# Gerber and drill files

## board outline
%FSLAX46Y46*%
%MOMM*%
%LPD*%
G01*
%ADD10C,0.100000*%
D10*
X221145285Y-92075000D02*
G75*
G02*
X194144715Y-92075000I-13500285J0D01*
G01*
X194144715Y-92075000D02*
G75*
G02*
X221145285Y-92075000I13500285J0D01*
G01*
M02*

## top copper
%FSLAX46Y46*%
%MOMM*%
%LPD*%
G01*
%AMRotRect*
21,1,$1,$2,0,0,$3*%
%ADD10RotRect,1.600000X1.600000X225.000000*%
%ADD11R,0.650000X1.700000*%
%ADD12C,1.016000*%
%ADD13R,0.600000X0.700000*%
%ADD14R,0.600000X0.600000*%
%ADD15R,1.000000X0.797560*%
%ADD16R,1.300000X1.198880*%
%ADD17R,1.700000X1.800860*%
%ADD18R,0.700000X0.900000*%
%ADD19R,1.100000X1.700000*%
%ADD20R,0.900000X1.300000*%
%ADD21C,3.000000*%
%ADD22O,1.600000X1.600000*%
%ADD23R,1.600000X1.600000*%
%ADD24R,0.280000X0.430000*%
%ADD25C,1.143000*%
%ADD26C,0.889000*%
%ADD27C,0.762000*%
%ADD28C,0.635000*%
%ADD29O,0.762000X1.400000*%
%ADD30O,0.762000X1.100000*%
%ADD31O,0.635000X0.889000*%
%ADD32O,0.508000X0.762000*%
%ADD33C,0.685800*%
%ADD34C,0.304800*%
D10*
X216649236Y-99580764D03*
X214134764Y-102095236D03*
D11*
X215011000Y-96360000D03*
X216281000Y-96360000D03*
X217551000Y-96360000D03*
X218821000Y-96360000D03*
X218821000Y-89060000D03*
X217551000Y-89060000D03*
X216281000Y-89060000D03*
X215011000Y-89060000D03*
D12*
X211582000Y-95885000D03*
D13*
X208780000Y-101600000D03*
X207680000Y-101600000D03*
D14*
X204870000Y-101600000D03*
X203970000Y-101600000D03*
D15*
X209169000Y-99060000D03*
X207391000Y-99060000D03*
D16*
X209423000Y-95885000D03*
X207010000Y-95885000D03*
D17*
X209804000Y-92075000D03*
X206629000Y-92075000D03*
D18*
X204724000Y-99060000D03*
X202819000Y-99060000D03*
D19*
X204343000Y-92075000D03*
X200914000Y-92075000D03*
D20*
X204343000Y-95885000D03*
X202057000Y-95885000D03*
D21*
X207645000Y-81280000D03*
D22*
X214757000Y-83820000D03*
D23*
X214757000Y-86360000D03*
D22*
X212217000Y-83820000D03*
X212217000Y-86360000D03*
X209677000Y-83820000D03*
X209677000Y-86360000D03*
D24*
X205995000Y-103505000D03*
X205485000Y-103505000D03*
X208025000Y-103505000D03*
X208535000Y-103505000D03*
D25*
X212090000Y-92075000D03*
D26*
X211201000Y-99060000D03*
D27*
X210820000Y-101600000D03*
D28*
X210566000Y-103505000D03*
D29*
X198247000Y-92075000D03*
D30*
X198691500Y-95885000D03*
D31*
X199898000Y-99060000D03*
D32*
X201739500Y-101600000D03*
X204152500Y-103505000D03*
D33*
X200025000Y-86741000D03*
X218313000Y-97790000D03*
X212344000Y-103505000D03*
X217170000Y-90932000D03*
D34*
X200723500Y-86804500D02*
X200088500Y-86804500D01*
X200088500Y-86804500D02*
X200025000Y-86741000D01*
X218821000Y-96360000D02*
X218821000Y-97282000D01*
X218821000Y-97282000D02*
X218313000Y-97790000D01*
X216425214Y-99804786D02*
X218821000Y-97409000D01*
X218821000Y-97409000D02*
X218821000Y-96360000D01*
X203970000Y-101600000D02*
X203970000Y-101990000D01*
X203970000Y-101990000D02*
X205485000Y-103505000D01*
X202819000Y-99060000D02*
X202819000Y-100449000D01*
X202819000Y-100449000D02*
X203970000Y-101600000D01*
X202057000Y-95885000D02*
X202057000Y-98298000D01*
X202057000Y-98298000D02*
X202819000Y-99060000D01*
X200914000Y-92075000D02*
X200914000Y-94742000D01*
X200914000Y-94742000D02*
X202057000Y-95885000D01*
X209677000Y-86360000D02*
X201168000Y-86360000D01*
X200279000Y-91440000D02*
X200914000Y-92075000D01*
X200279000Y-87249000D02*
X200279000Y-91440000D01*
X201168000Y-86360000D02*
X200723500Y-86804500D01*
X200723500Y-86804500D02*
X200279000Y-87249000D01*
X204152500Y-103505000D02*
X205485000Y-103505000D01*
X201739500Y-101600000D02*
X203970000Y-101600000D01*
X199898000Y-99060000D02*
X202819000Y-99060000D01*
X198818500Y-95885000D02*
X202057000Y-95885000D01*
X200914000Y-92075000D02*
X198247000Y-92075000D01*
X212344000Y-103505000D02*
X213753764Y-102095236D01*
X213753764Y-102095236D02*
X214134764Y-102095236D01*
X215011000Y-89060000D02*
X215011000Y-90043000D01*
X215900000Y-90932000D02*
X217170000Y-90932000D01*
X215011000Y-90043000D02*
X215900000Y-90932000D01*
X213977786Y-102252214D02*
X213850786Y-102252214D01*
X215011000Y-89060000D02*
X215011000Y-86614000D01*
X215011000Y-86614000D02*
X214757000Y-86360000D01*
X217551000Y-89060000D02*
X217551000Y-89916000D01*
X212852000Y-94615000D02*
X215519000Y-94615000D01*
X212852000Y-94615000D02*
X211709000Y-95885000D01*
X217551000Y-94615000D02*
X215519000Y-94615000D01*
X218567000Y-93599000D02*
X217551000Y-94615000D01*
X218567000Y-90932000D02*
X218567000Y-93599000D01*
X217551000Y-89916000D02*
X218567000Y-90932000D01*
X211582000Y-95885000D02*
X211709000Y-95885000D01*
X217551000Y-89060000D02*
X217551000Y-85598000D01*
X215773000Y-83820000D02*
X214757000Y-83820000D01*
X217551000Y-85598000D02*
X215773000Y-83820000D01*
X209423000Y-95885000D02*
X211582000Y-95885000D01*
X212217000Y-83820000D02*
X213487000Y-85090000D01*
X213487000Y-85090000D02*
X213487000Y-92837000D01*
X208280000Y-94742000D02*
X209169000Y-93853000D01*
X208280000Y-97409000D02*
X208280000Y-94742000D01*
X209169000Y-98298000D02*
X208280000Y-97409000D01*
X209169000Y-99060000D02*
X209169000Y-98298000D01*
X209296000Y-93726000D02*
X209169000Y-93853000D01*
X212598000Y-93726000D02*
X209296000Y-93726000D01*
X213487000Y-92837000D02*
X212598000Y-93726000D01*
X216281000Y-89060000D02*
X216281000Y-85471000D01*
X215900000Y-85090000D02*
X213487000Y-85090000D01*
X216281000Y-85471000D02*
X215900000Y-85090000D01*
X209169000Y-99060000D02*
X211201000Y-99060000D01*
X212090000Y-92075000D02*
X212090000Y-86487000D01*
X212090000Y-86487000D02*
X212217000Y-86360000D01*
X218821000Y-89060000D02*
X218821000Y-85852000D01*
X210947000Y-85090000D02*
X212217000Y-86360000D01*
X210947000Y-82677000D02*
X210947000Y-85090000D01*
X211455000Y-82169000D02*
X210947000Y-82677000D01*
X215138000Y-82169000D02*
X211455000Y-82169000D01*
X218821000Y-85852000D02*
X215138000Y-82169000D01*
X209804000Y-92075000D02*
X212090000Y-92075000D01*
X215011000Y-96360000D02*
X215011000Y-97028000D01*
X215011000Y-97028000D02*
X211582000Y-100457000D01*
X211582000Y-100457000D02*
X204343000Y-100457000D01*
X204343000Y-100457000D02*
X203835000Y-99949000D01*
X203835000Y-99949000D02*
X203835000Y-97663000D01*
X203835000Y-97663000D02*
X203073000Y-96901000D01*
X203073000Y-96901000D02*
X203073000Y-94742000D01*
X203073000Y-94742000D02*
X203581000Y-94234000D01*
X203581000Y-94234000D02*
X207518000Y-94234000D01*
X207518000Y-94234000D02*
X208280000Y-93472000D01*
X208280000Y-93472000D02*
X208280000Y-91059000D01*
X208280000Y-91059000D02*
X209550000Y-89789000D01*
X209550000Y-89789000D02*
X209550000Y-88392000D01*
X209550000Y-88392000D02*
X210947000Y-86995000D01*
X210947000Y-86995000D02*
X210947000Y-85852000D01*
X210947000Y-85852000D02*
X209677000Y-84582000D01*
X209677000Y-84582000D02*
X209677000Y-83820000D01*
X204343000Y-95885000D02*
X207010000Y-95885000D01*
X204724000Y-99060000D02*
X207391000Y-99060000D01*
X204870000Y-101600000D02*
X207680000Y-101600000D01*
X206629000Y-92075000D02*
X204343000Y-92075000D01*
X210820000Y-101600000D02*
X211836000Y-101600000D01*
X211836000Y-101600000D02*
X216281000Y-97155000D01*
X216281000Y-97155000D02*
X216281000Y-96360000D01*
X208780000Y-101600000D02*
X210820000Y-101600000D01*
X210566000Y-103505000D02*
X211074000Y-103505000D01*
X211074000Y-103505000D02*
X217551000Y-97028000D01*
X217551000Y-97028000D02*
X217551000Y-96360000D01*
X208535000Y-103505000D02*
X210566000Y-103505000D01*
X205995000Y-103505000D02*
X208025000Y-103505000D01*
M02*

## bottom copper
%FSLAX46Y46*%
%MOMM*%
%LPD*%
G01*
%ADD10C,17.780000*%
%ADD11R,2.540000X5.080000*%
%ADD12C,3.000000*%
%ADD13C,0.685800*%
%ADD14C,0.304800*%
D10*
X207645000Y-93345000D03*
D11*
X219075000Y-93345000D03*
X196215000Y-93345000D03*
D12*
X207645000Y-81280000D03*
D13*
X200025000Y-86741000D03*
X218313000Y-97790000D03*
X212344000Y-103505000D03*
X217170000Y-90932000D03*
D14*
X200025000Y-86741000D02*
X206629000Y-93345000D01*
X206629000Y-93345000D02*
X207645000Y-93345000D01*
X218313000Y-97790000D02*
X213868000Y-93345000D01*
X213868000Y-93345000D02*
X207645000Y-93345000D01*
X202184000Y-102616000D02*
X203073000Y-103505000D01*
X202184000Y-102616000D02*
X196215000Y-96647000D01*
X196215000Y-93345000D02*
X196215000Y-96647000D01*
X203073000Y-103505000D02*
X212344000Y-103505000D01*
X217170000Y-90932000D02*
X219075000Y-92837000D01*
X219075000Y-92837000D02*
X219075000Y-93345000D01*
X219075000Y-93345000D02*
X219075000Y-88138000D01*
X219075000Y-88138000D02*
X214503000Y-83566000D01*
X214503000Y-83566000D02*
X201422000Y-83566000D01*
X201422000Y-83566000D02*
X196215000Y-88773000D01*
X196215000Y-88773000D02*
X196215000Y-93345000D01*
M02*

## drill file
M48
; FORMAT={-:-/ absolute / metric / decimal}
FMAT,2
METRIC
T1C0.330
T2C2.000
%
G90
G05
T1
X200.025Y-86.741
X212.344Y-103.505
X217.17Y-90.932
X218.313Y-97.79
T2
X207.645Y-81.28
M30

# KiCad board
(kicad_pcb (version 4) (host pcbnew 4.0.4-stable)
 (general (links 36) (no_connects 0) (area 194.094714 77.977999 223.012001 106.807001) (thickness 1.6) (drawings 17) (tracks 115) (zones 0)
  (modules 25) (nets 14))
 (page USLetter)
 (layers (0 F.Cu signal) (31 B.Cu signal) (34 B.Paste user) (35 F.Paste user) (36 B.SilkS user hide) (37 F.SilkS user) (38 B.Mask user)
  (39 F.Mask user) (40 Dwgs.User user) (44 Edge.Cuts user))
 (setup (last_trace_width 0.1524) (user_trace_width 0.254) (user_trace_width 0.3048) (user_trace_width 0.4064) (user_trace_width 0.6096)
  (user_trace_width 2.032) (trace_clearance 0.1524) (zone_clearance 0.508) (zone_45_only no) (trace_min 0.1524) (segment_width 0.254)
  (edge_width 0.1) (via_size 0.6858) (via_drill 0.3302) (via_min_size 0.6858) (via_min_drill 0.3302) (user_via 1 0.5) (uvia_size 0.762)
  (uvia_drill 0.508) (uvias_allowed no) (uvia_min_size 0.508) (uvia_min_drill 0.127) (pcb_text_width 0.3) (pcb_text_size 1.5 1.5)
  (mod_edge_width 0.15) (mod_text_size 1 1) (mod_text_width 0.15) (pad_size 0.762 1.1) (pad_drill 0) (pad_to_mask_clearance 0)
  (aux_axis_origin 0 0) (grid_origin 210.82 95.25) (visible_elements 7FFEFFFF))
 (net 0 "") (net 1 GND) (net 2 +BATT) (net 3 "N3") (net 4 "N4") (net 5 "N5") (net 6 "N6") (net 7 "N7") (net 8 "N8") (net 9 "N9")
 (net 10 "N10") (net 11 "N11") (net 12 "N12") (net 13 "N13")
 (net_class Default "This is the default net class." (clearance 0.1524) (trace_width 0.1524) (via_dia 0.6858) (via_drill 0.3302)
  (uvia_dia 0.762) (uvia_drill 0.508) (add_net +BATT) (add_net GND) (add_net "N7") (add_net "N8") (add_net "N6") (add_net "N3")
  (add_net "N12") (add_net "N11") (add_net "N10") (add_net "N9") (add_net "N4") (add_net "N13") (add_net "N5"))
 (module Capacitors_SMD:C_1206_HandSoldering (layer F.Cu) (at 215.392 100.838 225)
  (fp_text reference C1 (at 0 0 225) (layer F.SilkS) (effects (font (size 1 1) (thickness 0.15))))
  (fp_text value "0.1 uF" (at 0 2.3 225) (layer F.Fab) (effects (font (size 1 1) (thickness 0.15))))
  (pad 1 smd rect (at -1.778 0 225) (size 1.6 1.6) (layers F.Cu F.Paste F.Mask) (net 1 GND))
  (pad 2 smd rect (at 1.778 0 225) (size 1.6 1.6) (layers F.Cu F.Paste F.Mask) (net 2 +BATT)))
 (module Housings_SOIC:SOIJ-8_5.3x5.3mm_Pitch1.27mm (layer F.Cu) (at 216.916 92.71 90)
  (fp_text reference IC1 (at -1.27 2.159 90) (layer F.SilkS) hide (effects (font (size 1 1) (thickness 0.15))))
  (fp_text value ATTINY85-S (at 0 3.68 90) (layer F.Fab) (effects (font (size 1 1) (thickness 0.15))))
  (pad 1 smd rect (at -3.65 -1.905 90) (size 1.7 0.65) (layers F.Cu F.Paste F.Mask) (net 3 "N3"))
  (pad 2 smd rect (at -3.65 -0.635 90) (size 1.7 0.65) (layers F.Cu F.Paste F.Mask) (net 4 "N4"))
  (pad 3 smd rect (at -3.65 0.635 90) (size 1.7 0.65) (layers F.Cu F.Paste F.Mask) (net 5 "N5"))
  (pad 4 smd rect (at -3.65 1.905 90) (size 1.7 0.65) (layers F.Cu F.Paste F.Mask) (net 1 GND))
  (pad 5 smd rect (at 3.65 1.905 90) (size 1.7 0.65) (layers F.Cu F.Paste F.Mask) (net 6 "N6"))
  (pad 6 smd rect (at 3.65 0.635 90) (size 1.7 0.65) (layers F.Cu F.Paste F.Mask) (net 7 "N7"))
  (pad 7 smd rect (at 3.65 -0.635 90) (size 1.7 0.65) (layers F.Cu F.Paste F.Mask) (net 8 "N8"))
  (pad 8 smd rect (at 3.65 -1.905 90) (size 1.7 0.65) (layers F.Cu F.Paste F.Mask) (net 2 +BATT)))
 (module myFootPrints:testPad (layer F.Cu) (at 211.582 95.885)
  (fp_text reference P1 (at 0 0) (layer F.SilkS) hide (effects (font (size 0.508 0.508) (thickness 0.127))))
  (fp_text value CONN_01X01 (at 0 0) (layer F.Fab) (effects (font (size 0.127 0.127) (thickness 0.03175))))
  (pad 1 smd circle (at 0 0) (size 1.016 1.016) (layers F.Cu F.Paste F.Mask) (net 7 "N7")))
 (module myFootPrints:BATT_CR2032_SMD (layer B.Cu) (at 207.645 93.345 180)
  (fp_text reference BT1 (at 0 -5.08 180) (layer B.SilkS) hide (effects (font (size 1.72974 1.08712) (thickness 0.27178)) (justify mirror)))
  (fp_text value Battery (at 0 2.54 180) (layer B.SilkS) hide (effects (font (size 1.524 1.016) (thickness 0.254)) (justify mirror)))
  (pad 2 smd circle (at 0 0 180) (size 17.78 17.78) (layers B.Cu B.Paste B.Mask) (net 1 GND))
  (pad 1 smd rect (at -11.43 0 180) (size 2.54 5.08) (layers B.Cu B.Paste B.Mask) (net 2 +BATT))
  (pad 1 smd rect (at 11.43 0 180) (size 2.54 5.08) (layers B.Cu B.Paste B.Mask) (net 2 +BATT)))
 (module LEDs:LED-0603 (layer F.Cu) (at 208.28 101.6)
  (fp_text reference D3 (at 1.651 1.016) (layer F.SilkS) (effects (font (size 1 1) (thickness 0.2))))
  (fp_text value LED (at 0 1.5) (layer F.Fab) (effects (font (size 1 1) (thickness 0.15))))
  (pad 2 smd rect (at 0.5 0 180) (size 0.6 0.7) (layers F.Cu F.Paste F.Mask) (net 4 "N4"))
  (pad 1 smd rect (at -0.6 0 180) (size 0.6 0.7) (layers F.Cu F.Paste F.Mask) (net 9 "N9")))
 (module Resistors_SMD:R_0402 (layer F.Cu) (at 204.47 101.6 180)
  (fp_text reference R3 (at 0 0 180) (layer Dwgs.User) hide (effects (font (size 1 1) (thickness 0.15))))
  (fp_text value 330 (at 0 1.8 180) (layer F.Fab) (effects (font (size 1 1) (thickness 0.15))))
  (pad 1 smd rect (at -0.4 0 180) (size 0.6 0.6) (layers F.Cu F.Paste F.Mask) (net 9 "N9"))
  (pad 2 smd rect (at 0.5 0 180) (size 0.6 0.6) (layers F.Cu F.Paste F.Mask) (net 1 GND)))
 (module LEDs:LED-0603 (layer F.Cu) (at 208.28 99.06)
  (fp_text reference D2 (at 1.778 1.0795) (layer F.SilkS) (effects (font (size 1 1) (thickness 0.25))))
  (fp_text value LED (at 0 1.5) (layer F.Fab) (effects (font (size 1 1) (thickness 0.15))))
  (pad 2 smd rect (at 0.889 0 180) (size 1 0.79756) (layers F.Cu F.Paste F.Mask) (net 8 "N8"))
  (pad 1 smd rect (at -0.889 0 180) (size 1 0.79756) (layers F.Cu F.Paste F.Mask) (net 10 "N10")))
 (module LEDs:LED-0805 (layer F.Cu) (at 208.28 95.885)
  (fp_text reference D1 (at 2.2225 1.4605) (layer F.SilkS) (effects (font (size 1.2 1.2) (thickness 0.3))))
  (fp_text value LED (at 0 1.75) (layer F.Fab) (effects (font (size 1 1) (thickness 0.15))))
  (pad 2 smd rect (at 1.143 0 180) (size 1.3 1.19888) (layers F.Cu F.Paste F.Mask) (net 7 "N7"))
  (pad 1 smd rect (at -1.27 0 180) (size 1.3 1.19888) (layers F.Cu F.Paste F.Mask) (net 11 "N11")))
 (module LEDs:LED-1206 (layer F.Cu) (at 208.28 92.075)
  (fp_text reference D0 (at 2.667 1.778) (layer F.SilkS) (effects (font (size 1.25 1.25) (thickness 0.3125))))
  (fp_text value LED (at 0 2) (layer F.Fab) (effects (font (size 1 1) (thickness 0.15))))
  (pad 2 smd rect (at 1.524 0 180) (size 1.7 1.80086) (layers F.Cu F.Paste F.Mask) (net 6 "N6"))
  (pad 1 smd rect (at -1.651 0 180) (size 1.7 1.80086) (layers F.Cu F.Paste F.Mask) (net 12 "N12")))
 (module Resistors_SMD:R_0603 (layer F.Cu) (at 203.835 99.06 180)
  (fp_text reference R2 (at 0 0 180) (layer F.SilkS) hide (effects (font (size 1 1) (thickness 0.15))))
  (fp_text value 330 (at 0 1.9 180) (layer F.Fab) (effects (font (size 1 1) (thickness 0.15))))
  (pad 1 smd rect (at -0.889 0 180) (size 0.7 0.9) (layers F.Cu F.Paste F.Mask) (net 10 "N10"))
  (pad 2 smd rect (at 1.016 0 180) (size 0.7 0.9) (layers F.Cu F.Paste F.Mask) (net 1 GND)))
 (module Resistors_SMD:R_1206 (layer F.Cu) (at 202.565 92.075 180)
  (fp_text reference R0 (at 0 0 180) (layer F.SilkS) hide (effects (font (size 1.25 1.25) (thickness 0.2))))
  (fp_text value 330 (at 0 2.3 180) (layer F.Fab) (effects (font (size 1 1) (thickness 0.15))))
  (pad 1 smd rect (at -1.778 0 180) (size 1.1 1.7) (layers F.Cu F.Paste F.Mask) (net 12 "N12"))
  (pad 2 smd rect (at 1.651 0 180) (size 1.1 1.7) (layers F.Cu F.Paste F.Mask) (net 1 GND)))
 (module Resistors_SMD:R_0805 (layer F.Cu) (at 203.2 95.885 180)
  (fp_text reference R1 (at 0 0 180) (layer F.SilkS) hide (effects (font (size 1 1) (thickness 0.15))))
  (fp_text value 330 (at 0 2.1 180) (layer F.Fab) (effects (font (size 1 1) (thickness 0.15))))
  (pad 1 smd rect (at -1.143 0 180) (size 0.9 1.3) (layers F.Cu F.Paste F.Mask) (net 11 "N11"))
  (pad 2 smd rect (at 1.143 0 180) (size 0.9 1.3) (layers F.Cu F.Paste F.Mask) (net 1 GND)))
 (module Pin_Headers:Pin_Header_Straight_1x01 (layer F.Cu) (at 207.645 81.28)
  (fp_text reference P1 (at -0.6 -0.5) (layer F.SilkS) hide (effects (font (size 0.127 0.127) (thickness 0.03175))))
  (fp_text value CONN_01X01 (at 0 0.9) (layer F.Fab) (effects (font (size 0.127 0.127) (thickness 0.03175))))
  (pad P5 thru_hole circle (at 0 0) (size 3 3) (drill 2) (layers *.Cu *.Mask)))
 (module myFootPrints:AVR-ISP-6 (layer F.Cu) (at 214.757 83.82 270)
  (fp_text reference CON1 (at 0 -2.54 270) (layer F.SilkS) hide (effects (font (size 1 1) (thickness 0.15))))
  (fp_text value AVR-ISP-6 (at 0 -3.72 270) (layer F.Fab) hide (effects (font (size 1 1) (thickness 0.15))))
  (pad 1 smd oval (at 0 0 270) (size 1.6 1.6) (layers F.Cu F.Paste F.Mask) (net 7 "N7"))
  (pad 2 smd rect (at 2.54 0 270) (size 1.6 1.6) (layers F.Cu F.Paste F.Mask) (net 2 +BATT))
  (pad 3 smd oval (at 0 2.54 270) (size 1.6 1.6) (layers F.Cu F.Paste F.Mask) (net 8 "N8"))
  (pad 4 smd oval (at 2.54 2.54 270) (size 1.6 1.6) (layers F.Cu F.Paste F.Mask) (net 6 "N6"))
  (pad 5 smd oval (at 0 5.08 270) (size 1.6 1.6) (layers F.Cu F.Paste F.Mask) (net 3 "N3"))
  (pad 6 smd oval (at 2.54 5.08 270) (size 1.6 1.6) (layers F.Cu F.Paste F.Mask) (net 1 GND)))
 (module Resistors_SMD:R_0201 (layer F.Cu) (at 205.74 103.505 180)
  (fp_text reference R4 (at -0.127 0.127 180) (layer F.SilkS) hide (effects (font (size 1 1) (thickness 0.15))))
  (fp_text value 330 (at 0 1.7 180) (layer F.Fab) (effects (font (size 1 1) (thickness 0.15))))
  (pad 1 smd rect (at -0.255 0 180) (size 0.28 0.43) (layers F.Cu F.Paste F.Mask) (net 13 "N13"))
  (pad 2 smd rect (at 0.255 0 180) (size 0.28 0.43) (layers F.Cu F.Paste F.Mask) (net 1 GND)))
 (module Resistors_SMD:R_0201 (layer F.Cu) (at 208.28 103.505)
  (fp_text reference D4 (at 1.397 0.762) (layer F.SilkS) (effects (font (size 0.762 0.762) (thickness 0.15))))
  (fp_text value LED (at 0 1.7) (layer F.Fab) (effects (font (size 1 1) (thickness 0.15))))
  (pad 1 smd rect (at -0.255 0) (size 0.28 0.43) (layers F.Cu F.Paste F.Mask) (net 13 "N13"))
  (pad 2 smd rect (at 0.255 0) (size 0.28 0.43) (layers F.Cu F.Paste F.Mask) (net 5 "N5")))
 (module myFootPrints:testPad (layer F.Cu) (at 212.09 92.075)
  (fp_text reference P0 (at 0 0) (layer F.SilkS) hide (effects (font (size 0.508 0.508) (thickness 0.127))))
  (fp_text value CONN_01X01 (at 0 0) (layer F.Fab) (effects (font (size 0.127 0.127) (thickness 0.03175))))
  (pad 1 smd circle (at 0 0) (size 1.143 1.143) (layers F.Cu F.Paste F.Mask) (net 6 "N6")))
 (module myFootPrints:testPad (layer F.Cu) (at 211.201 99.06)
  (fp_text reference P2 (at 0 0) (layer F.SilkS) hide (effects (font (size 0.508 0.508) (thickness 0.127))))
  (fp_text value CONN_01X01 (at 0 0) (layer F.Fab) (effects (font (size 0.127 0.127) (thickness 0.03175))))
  (pad 1 smd circle (at 0 0) (size 0.889 0.889) (layers F.Cu F.Paste F.Mask) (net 8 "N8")))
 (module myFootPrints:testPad (layer F.Cu) (at 210.82 101.6)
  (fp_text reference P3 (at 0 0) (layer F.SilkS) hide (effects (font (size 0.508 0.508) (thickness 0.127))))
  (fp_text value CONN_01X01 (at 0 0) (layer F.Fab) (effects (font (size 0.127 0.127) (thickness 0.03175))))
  (pad 1 smd circle (at 0 0) (size 0.762 0.762) (layers F.Cu F.Paste F.Mask) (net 4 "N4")))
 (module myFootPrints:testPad (layer F.Cu) (at 210.566 103.505)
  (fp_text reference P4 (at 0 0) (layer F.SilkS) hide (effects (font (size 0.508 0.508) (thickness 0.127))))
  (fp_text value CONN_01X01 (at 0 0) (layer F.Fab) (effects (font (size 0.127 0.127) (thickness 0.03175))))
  (pad 1 smd circle (at 0 0) (size 0.635 0.635) (layers F.Cu F.Paste F.Mask) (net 5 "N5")))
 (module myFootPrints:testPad (layer F.Cu) (at 198.247 92.075)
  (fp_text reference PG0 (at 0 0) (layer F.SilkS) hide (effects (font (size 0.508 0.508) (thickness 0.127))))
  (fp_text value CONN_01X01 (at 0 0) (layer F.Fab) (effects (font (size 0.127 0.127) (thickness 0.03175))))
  (pad 1 smd oval (at 0 0) (size 0.762 1.4) (layers F.Cu F.Paste F.Mask) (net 1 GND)))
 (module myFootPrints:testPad (layer F.Cu) (at 198.6915 95.885)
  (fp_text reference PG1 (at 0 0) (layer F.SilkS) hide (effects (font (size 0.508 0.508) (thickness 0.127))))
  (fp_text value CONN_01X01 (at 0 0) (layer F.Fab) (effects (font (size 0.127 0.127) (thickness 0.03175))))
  (pad 1 smd oval (at 0 0) (size 0.762 1.1) (layers F.Cu F.Paste F.Mask) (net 1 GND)))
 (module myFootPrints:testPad (layer F.Cu) (at 199.898 99.06)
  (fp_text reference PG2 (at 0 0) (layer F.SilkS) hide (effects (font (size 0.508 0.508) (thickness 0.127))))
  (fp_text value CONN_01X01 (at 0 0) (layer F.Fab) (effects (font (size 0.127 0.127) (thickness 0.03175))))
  (pad 1 smd oval (at 0 0) (size 0.635 0.889) (layers F.Cu F.Paste F.Mask) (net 1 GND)))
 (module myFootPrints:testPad (layer F.Cu) (at 201.7395 101.6)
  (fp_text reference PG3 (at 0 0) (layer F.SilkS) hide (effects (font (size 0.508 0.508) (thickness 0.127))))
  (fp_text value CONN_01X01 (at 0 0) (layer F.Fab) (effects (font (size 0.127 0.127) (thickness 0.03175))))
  (pad 1 smd oval (at 0 0) (size 0.508 0.762) (layers F.Cu F.Paste F.Mask) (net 1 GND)))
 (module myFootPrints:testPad (layer F.Cu) (at 204.1525 103.505)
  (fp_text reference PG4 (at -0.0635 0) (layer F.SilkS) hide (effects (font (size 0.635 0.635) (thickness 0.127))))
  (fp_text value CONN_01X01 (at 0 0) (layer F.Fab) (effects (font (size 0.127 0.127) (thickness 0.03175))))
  (pad 1 smd oval (at 0 0) (size 0.508 0.762) (layers F.Cu F.Paste F.Mask) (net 1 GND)))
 (gr_circle (center 207.645 92.075) (end 197.485 83.185) (layer Edge.Cuts) (width 0.1))
 (segment (start 200.7235 86.8045) (end 200.0885 86.8045) (width 0.3048) (layer F.Cu) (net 1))
 (segment (start 200.025 86.741) (end 206.629 93.345) (width 0.3048) (layer B.Cu) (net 1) (status 20))
 (via (at 200.025 86.741) (size 0.6858) (drill 0.3302) (layers F.Cu B.Cu) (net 1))
 (segment (start 200.0885 86.8045) (end 200.025 86.741) (width 0.3048) (layer F.Cu) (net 1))
 (segment (start 206.629 93.345) (end 207.645 93.345) (width 0.3048) (layer B.Cu) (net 1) (status 30))
 (segment (start 218.821 96.36) (end 218.821 97.282) (width 0.3048) (layer F.Cu) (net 1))
 (segment (start 218.313 97.79) (end 213.868 93.345) (width 0.3048) (layer B.Cu) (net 1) (status 20))
 (via (at 218.313 97.79) (size 0.6858) (drill 0.3302) (layers F.Cu B.Cu) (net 1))
 (segment (start 218.821 97.282) (end 218.313 97.79) (width 0.3048) (layer F.Cu) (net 1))
 (segment (start 213.868 93.345) (end 207.645 93.345) (width 0.3048) (layer B.Cu) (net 1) (status 30))
 (segment (start 216.425214 99.804786) (end 218.821 97.409) (width 0.3048) (layer F.Cu) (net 1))
 (segment (start 218.821 97.409) (end 218.821 96.36) (width 0.3048) (layer F.Cu) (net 1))
 (segment (start 203.97 101.6) (end 203.97 101.99) (width 0.3048) (layer F.Cu) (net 1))
 (segment (start 203.97 101.99) (end 205.485 103.505) (width 0.3048) (layer F.Cu) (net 1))
 (segment (start 202.819 99.06) (end 202.819 100.449) (width 0.3048) (layer F.Cu) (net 1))
 (segment (start 202.819 100.449) (end 203.97 101.6) (width 0.3048) (layer F.Cu) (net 1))
 (segment (start 202.057 95.885) (end 202.057 98.298) (width 0.3048) (layer F.Cu) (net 1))
 (segment (start 202.057 98.298) (end 202.819 99.06) (width 0.3048) (layer F.Cu) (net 1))
 (segment (start 200.914 92.075) (end 200.914 94.742) (width 0.3048) (layer F.Cu) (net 1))
 (segment (start 200.914 94.742) (end 202.057 95.885) (width 0.3048) (layer F.Cu) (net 1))
 (segment (start 209.677 86.36) (end 201.168 86.36) (width 0.3048) (layer F.Cu) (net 1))
 (segment (start 200.279 91.44) (end 200.914 92.075) (width 0.3048) (layer F.Cu) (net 1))
 (segment (start 200.279 87.249) (end 200.279 91.44) (width 0.3048) (layer F.Cu) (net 1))
 (segment (start 201.168 86.36) (end 200.7235 86.8045) (width 0.3048) (layer F.Cu) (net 1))
 (segment (start 200.7235 86.8045) (end 200.279 87.249) (width 0.3048) (layer F.Cu) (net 1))
 (segment (start 204.1525 103.505) (end 205.485 103.505) (width 0.3048) (layer F.Cu) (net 1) (status 10))
 (segment (start 201.7395 101.6) (end 203.97 101.6) (width 0.3048) (layer F.Cu) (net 1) (status 10))
 (segment (start 199.898 99.06) (end 202.819 99.06) (width 0.3048) (layer F.Cu) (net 1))
 (segment (start 198.8185 95.885) (end 202.057 95.885) (width 0.3048) (layer F.Cu) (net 1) (status 10))
 (segment (start 200.914 92.075) (end 198.247 92.075) (width 0.3048) (layer F.Cu) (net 1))
 (segment (start 202.184 102.616) (end 203.073 103.505) (width 0.3048) (layer B.Cu) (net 2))
 (segment (start 202.184 102.616) (end 196.215 96.647) (width 0.3048) (layer B.Cu) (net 2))
 (segment (start 196.215 93.345) (end 196.215 96.647) (width 0.3048) (layer B.Cu) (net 2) (status 10))
 (segment (start 212.344 103.505) (end 213.753764 102.095236) (width 0.3048) (layer F.Cu) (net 2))
 (via (at 212.344 103.505) (size 0.6858) (drill 0.3302) (layers F.Cu B.Cu) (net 2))
 (segment (start 203.073 103.505) (end 212.344 103.505) (width 0.3048) (layer B.Cu) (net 2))
 (segment (start 213.753764 102.095236) (end 214.134764 102.095236) (width 0.3048) (layer F.Cu) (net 2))
 (segment (start 215.011 89.06) (end 215.011 90.043) (width 0.3048) (layer F.Cu) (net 2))
 (segment (start 217.17 90.932) (end 219.075 92.837) (width 0.3048) (layer B.Cu) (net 2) (status 20))
 (via (at 217.17 90.932) (size 0.6858) (drill 0.3302) (layers F.Cu B.Cu) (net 2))
 (segment (start 215.9 90.932) (end 217.17 90.932) (width 0.3048) (layer F.Cu) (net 2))
 (segment (start 215.011 90.043) (end 215.9 90.932) (width 0.3048) (layer F.Cu) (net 2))
 (segment (start 219.075 92.837) (end 219.075 93.345) (width 0.3048) (layer B.Cu) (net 2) (status 30))
 (segment (start 219.075 93.345) (end 219.075 88.138) (width 0.3048) (layer B.Cu) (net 2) (status 10))
 (segment (start 219.075 88.138) (end 214.503 83.566) (width 0.3048) (layer B.Cu) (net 2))
 (segment (start 214.503 83.566) (end 201.422 83.566) (width 0.3048) (layer B.Cu) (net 2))
 (segment (start 201.422 83.566) (end 196.215 88.773) (width 0.3048) (layer B.Cu) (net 2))
 (segment (start 196.215 88.773) (end 196.215 93.345) (width 0.3048) (layer B.Cu) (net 2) (status 20))
 (segment (start 213.977786 102.252214) (end 213.850786 102.252214) (width 0.3048) (layer F.Cu) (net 2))
 (segment (start 215.011 89.06) (end 215.011 86.614) (width 0.3048) (layer F.Cu) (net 2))
 (segment (start 215.011 86.614) (end 214.757 86.36) (width 0.3048) (layer F.Cu) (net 2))
 (segment (start 217.551 89.06) (end 217.551 89.916) (width 0.3048) (layer F.Cu) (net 7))
 (segment (start 212.852 94.615) (end 215.519 94.615) (width 0.3048) (layer F.Cu) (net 7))
 (segment (start 212.852 94.615) (end 211.709 95.885) (width 0.3048) (layer F.Cu) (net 7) (status 20))
 (segment (start 217.551 94.615) (end 215.519 94.615) (width 0.3048) (layer F.Cu) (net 7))
 (segment (start 218.567 93.599) (end 217.551 94.615) (width 0.3048) (layer F.Cu) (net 7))
 (segment (start 218.567 90.932) (end 218.567 93.599) (width 0.3048) (layer F.Cu) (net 7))
 (segment (start 217.551 89.916) (end 218.567 90.932) (width 0.3048) (layer F.Cu) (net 7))
 (segment (start 211.582 95.885) (end 211.709 95.885) (width 0.3048) (layer F.Cu) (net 7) (status 30))
 (segment (start 217.551 89.06) (end 217.551 85.598) (width 0.3048) (layer F.Cu) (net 7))
 (segment (start 215.773 83.82) (end 214.757 83.82) (width 0.3048) (layer F.Cu) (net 7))
 (segment (start 217.551 85.598) (end 215.773 83.82) (width 0.3048) (layer F.Cu) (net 7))
 (segment (start 209.423 95.885) (end 211.582 95.885) (width 0.3048) (layer F.Cu) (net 7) (status 20))
 (segment (start 212.217 83.82) (end 213.487 85.09) (width 0.3048) (layer F.Cu) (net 8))
 (segment (start 213.487 85.09) (end 213.487 92.837) (width 0.3048) (layer F.Cu) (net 8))
 (segment (start 208.28 94.742) (end 209.169 93.853) (width 0.3048) (layer F.Cu) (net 8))
 (segment (start 208.28 97.409) (end 208.28 94.742) (width 0.3048) (layer F.Cu) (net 8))
 (segment (start 209.169 98.298) (end 208.28 97.409) (width 0.3048) (layer F.Cu) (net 8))
 (segment (start 209.169 99.06) (end 209.169 98.298) (width 0.3048) (layer F.Cu) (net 8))
 (segment (start 209.296 93.726) (end 209.169 93.853) (width 0.3048) (layer F.Cu) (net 8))
 (segment (start 212.598 93.726) (end 209.296 93.726) (width 0.3048) (layer F.Cu) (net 8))
 (segment (start 213.487 92.837) (end 212.598 93.726) (width 0.3048) (layer F.Cu) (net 8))
 (segment (start 216.281 89.06) (end 216.281 85.471) (width 0.3048) (layer F.Cu) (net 8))
 (segment (start 215.9 85.09) (end 213.487 85.09) (width 0.3048) (layer F.Cu) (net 8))
 (segment (start 216.281 85.471) (end 215.9 85.09) (width 0.3048) (layer F.Cu) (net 8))
 (segment (start 209.169 99.06) (end 211.201 99.06) (width 0.3048) (layer F.Cu) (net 8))
 (segment (start 212.09 92.075) (end 212.09 86.487) (width 0.3048) (layer F.Cu) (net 6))
 (segment (start 212.09 86.487) (end 212.217 86.36) (width 0.3048) (layer F.Cu) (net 6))
 (segment (start 218.821 89.06) (end 218.821 85.852) (width 0.3048) (layer F.Cu) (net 6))
 (segment (start 210.947 85.09) (end 212.217 86.36) (width 0.3048) (layer F.Cu) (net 6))
 (segment (start 210.947 82.677) (end 210.947 85.09) (width 0.3048) (layer F.Cu) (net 6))
 (segment (start 211.455 82.169) (end 210.947 82.677) (width 0.3048) (layer F.Cu) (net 6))
 (segment (start 215.138 82.169) (end 211.455 82.169) (width 0.3048) (layer F.Cu) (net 6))
 (segment (start 218.821 85.852) (end 215.138 82.169) (width 0.3048) (layer F.Cu) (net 6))
 (segment (start 209.804 92.075) (end 212.09 92.075) (width 0.3048) (layer F.Cu) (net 6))
 (segment (start 215.011 96.36) (end 215.011 97.028) (width 0.3048) (layer F.Cu) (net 3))
 (segment (start 215.011 97.028) (end 211.582 100.457) (width 0.3048) (layer F.Cu) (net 3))
 (segment (start 211.582 100.457) (end 204.343 100.457) (width 0.3048) (layer F.Cu) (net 3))
 (segment (start 204.343 100.457) (end 203.835 99.949) (width 0.3048) (layer F.Cu) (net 3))
 (segment (start 203.835 99.949) (end 203.835 97.663) (width 0.3048) (layer F.Cu) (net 3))
 (segment (start 203.835 97.663) (end 203.073 96.901) (width 0.3048) (layer F.Cu) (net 3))
 (segment (start 203.073 96.901) (end 203.073 94.742) (width 0.3048) (layer F.Cu) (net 3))
 (segment (start 203.073 94.742) (end 203.581 94.234) (width 0.3048) (layer F.Cu) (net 3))
 (segment (start 203.581 94.234) (end 207.518 94.234) (width 0.3048) (layer F.Cu) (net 3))
 (segment (start 207.518 94.234) (end 208.28 93.472) (width 0.3048) (layer F.Cu) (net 3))
 (segment (start 208.28 93.472) (end 208.28 91.059) (width 0.3048) (layer F.Cu) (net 3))
 (segment (start 208.28 91.059) (end 209.55 89.789) (width 0.3048) (layer F.Cu) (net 3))
 (segment (start 209.55 89.789) (end 209.55 88.392) (width 0.3048) (layer F.Cu) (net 3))
 (segment (start 209.55 88.392) (end 210.947 86.995) (width 0.3048) (layer F.Cu) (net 3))
 (segment (start 210.947 86.995) (end 210.947 85.852) (width 0.3048) (layer F.Cu) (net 3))
 (segment (start 210.947 85.852) (end 209.677 84.582) (width 0.3048) (layer F.Cu) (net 3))
 (segment (start 209.677 84.582) (end 209.677 83.82) (width 0.3048) (layer F.Cu) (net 3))
 (segment (start 204.343 95.885) (end 207.01 95.885) (width 0.3048) (layer F.Cu) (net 11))
 (segment (start 204.724 99.06) (end 207.391 99.06) (width 0.3048) (layer F.Cu) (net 10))
 (segment (start 204.87 101.6) (end 207.68 101.6) (width 0.3048) (layer F.Cu) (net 9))
 (segment (start 206.629 92.075) (end 204.343 92.075) (width 0.3048) (layer F.Cu) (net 12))
 (segment (start 210.82 101.6) (end 211.836 101.6) (width 0.3048) (layer F.Cu) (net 4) (status 10))
 (segment (start 211.836 101.6) (end 216.281 97.155) (width 0.3048) (layer F.Cu) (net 4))
 (segment (start 216.281 97.155) (end 216.281 96.36) (width 0.3048) (layer F.Cu) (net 4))
 (segment (start 208.78 101.6) (end 210.82 101.6) (width 0.3048) (layer F.Cu) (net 4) (status 20))
 (segment (start 210.566 103.505) (end 211.074 103.505) (width 0.3048) (layer F.Cu) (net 5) (status 10))
 (segment (start 211.074 103.505) (end 217.551 97.028) (width 0.3048) (layer F.Cu) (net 5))
 (segment (start 217.551 97.028) (end 217.551 96.36) (width 0.3048) (layer F.Cu) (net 5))
 (segment (start 208.535 103.505) (end 210.566 103.505) (width 0.3048) (layer F.Cu) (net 5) (status 20))
 (segment (start 205.995 103.505) (end 208.025 103.505) (width 0.3048) (layer F.Cu) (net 13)))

